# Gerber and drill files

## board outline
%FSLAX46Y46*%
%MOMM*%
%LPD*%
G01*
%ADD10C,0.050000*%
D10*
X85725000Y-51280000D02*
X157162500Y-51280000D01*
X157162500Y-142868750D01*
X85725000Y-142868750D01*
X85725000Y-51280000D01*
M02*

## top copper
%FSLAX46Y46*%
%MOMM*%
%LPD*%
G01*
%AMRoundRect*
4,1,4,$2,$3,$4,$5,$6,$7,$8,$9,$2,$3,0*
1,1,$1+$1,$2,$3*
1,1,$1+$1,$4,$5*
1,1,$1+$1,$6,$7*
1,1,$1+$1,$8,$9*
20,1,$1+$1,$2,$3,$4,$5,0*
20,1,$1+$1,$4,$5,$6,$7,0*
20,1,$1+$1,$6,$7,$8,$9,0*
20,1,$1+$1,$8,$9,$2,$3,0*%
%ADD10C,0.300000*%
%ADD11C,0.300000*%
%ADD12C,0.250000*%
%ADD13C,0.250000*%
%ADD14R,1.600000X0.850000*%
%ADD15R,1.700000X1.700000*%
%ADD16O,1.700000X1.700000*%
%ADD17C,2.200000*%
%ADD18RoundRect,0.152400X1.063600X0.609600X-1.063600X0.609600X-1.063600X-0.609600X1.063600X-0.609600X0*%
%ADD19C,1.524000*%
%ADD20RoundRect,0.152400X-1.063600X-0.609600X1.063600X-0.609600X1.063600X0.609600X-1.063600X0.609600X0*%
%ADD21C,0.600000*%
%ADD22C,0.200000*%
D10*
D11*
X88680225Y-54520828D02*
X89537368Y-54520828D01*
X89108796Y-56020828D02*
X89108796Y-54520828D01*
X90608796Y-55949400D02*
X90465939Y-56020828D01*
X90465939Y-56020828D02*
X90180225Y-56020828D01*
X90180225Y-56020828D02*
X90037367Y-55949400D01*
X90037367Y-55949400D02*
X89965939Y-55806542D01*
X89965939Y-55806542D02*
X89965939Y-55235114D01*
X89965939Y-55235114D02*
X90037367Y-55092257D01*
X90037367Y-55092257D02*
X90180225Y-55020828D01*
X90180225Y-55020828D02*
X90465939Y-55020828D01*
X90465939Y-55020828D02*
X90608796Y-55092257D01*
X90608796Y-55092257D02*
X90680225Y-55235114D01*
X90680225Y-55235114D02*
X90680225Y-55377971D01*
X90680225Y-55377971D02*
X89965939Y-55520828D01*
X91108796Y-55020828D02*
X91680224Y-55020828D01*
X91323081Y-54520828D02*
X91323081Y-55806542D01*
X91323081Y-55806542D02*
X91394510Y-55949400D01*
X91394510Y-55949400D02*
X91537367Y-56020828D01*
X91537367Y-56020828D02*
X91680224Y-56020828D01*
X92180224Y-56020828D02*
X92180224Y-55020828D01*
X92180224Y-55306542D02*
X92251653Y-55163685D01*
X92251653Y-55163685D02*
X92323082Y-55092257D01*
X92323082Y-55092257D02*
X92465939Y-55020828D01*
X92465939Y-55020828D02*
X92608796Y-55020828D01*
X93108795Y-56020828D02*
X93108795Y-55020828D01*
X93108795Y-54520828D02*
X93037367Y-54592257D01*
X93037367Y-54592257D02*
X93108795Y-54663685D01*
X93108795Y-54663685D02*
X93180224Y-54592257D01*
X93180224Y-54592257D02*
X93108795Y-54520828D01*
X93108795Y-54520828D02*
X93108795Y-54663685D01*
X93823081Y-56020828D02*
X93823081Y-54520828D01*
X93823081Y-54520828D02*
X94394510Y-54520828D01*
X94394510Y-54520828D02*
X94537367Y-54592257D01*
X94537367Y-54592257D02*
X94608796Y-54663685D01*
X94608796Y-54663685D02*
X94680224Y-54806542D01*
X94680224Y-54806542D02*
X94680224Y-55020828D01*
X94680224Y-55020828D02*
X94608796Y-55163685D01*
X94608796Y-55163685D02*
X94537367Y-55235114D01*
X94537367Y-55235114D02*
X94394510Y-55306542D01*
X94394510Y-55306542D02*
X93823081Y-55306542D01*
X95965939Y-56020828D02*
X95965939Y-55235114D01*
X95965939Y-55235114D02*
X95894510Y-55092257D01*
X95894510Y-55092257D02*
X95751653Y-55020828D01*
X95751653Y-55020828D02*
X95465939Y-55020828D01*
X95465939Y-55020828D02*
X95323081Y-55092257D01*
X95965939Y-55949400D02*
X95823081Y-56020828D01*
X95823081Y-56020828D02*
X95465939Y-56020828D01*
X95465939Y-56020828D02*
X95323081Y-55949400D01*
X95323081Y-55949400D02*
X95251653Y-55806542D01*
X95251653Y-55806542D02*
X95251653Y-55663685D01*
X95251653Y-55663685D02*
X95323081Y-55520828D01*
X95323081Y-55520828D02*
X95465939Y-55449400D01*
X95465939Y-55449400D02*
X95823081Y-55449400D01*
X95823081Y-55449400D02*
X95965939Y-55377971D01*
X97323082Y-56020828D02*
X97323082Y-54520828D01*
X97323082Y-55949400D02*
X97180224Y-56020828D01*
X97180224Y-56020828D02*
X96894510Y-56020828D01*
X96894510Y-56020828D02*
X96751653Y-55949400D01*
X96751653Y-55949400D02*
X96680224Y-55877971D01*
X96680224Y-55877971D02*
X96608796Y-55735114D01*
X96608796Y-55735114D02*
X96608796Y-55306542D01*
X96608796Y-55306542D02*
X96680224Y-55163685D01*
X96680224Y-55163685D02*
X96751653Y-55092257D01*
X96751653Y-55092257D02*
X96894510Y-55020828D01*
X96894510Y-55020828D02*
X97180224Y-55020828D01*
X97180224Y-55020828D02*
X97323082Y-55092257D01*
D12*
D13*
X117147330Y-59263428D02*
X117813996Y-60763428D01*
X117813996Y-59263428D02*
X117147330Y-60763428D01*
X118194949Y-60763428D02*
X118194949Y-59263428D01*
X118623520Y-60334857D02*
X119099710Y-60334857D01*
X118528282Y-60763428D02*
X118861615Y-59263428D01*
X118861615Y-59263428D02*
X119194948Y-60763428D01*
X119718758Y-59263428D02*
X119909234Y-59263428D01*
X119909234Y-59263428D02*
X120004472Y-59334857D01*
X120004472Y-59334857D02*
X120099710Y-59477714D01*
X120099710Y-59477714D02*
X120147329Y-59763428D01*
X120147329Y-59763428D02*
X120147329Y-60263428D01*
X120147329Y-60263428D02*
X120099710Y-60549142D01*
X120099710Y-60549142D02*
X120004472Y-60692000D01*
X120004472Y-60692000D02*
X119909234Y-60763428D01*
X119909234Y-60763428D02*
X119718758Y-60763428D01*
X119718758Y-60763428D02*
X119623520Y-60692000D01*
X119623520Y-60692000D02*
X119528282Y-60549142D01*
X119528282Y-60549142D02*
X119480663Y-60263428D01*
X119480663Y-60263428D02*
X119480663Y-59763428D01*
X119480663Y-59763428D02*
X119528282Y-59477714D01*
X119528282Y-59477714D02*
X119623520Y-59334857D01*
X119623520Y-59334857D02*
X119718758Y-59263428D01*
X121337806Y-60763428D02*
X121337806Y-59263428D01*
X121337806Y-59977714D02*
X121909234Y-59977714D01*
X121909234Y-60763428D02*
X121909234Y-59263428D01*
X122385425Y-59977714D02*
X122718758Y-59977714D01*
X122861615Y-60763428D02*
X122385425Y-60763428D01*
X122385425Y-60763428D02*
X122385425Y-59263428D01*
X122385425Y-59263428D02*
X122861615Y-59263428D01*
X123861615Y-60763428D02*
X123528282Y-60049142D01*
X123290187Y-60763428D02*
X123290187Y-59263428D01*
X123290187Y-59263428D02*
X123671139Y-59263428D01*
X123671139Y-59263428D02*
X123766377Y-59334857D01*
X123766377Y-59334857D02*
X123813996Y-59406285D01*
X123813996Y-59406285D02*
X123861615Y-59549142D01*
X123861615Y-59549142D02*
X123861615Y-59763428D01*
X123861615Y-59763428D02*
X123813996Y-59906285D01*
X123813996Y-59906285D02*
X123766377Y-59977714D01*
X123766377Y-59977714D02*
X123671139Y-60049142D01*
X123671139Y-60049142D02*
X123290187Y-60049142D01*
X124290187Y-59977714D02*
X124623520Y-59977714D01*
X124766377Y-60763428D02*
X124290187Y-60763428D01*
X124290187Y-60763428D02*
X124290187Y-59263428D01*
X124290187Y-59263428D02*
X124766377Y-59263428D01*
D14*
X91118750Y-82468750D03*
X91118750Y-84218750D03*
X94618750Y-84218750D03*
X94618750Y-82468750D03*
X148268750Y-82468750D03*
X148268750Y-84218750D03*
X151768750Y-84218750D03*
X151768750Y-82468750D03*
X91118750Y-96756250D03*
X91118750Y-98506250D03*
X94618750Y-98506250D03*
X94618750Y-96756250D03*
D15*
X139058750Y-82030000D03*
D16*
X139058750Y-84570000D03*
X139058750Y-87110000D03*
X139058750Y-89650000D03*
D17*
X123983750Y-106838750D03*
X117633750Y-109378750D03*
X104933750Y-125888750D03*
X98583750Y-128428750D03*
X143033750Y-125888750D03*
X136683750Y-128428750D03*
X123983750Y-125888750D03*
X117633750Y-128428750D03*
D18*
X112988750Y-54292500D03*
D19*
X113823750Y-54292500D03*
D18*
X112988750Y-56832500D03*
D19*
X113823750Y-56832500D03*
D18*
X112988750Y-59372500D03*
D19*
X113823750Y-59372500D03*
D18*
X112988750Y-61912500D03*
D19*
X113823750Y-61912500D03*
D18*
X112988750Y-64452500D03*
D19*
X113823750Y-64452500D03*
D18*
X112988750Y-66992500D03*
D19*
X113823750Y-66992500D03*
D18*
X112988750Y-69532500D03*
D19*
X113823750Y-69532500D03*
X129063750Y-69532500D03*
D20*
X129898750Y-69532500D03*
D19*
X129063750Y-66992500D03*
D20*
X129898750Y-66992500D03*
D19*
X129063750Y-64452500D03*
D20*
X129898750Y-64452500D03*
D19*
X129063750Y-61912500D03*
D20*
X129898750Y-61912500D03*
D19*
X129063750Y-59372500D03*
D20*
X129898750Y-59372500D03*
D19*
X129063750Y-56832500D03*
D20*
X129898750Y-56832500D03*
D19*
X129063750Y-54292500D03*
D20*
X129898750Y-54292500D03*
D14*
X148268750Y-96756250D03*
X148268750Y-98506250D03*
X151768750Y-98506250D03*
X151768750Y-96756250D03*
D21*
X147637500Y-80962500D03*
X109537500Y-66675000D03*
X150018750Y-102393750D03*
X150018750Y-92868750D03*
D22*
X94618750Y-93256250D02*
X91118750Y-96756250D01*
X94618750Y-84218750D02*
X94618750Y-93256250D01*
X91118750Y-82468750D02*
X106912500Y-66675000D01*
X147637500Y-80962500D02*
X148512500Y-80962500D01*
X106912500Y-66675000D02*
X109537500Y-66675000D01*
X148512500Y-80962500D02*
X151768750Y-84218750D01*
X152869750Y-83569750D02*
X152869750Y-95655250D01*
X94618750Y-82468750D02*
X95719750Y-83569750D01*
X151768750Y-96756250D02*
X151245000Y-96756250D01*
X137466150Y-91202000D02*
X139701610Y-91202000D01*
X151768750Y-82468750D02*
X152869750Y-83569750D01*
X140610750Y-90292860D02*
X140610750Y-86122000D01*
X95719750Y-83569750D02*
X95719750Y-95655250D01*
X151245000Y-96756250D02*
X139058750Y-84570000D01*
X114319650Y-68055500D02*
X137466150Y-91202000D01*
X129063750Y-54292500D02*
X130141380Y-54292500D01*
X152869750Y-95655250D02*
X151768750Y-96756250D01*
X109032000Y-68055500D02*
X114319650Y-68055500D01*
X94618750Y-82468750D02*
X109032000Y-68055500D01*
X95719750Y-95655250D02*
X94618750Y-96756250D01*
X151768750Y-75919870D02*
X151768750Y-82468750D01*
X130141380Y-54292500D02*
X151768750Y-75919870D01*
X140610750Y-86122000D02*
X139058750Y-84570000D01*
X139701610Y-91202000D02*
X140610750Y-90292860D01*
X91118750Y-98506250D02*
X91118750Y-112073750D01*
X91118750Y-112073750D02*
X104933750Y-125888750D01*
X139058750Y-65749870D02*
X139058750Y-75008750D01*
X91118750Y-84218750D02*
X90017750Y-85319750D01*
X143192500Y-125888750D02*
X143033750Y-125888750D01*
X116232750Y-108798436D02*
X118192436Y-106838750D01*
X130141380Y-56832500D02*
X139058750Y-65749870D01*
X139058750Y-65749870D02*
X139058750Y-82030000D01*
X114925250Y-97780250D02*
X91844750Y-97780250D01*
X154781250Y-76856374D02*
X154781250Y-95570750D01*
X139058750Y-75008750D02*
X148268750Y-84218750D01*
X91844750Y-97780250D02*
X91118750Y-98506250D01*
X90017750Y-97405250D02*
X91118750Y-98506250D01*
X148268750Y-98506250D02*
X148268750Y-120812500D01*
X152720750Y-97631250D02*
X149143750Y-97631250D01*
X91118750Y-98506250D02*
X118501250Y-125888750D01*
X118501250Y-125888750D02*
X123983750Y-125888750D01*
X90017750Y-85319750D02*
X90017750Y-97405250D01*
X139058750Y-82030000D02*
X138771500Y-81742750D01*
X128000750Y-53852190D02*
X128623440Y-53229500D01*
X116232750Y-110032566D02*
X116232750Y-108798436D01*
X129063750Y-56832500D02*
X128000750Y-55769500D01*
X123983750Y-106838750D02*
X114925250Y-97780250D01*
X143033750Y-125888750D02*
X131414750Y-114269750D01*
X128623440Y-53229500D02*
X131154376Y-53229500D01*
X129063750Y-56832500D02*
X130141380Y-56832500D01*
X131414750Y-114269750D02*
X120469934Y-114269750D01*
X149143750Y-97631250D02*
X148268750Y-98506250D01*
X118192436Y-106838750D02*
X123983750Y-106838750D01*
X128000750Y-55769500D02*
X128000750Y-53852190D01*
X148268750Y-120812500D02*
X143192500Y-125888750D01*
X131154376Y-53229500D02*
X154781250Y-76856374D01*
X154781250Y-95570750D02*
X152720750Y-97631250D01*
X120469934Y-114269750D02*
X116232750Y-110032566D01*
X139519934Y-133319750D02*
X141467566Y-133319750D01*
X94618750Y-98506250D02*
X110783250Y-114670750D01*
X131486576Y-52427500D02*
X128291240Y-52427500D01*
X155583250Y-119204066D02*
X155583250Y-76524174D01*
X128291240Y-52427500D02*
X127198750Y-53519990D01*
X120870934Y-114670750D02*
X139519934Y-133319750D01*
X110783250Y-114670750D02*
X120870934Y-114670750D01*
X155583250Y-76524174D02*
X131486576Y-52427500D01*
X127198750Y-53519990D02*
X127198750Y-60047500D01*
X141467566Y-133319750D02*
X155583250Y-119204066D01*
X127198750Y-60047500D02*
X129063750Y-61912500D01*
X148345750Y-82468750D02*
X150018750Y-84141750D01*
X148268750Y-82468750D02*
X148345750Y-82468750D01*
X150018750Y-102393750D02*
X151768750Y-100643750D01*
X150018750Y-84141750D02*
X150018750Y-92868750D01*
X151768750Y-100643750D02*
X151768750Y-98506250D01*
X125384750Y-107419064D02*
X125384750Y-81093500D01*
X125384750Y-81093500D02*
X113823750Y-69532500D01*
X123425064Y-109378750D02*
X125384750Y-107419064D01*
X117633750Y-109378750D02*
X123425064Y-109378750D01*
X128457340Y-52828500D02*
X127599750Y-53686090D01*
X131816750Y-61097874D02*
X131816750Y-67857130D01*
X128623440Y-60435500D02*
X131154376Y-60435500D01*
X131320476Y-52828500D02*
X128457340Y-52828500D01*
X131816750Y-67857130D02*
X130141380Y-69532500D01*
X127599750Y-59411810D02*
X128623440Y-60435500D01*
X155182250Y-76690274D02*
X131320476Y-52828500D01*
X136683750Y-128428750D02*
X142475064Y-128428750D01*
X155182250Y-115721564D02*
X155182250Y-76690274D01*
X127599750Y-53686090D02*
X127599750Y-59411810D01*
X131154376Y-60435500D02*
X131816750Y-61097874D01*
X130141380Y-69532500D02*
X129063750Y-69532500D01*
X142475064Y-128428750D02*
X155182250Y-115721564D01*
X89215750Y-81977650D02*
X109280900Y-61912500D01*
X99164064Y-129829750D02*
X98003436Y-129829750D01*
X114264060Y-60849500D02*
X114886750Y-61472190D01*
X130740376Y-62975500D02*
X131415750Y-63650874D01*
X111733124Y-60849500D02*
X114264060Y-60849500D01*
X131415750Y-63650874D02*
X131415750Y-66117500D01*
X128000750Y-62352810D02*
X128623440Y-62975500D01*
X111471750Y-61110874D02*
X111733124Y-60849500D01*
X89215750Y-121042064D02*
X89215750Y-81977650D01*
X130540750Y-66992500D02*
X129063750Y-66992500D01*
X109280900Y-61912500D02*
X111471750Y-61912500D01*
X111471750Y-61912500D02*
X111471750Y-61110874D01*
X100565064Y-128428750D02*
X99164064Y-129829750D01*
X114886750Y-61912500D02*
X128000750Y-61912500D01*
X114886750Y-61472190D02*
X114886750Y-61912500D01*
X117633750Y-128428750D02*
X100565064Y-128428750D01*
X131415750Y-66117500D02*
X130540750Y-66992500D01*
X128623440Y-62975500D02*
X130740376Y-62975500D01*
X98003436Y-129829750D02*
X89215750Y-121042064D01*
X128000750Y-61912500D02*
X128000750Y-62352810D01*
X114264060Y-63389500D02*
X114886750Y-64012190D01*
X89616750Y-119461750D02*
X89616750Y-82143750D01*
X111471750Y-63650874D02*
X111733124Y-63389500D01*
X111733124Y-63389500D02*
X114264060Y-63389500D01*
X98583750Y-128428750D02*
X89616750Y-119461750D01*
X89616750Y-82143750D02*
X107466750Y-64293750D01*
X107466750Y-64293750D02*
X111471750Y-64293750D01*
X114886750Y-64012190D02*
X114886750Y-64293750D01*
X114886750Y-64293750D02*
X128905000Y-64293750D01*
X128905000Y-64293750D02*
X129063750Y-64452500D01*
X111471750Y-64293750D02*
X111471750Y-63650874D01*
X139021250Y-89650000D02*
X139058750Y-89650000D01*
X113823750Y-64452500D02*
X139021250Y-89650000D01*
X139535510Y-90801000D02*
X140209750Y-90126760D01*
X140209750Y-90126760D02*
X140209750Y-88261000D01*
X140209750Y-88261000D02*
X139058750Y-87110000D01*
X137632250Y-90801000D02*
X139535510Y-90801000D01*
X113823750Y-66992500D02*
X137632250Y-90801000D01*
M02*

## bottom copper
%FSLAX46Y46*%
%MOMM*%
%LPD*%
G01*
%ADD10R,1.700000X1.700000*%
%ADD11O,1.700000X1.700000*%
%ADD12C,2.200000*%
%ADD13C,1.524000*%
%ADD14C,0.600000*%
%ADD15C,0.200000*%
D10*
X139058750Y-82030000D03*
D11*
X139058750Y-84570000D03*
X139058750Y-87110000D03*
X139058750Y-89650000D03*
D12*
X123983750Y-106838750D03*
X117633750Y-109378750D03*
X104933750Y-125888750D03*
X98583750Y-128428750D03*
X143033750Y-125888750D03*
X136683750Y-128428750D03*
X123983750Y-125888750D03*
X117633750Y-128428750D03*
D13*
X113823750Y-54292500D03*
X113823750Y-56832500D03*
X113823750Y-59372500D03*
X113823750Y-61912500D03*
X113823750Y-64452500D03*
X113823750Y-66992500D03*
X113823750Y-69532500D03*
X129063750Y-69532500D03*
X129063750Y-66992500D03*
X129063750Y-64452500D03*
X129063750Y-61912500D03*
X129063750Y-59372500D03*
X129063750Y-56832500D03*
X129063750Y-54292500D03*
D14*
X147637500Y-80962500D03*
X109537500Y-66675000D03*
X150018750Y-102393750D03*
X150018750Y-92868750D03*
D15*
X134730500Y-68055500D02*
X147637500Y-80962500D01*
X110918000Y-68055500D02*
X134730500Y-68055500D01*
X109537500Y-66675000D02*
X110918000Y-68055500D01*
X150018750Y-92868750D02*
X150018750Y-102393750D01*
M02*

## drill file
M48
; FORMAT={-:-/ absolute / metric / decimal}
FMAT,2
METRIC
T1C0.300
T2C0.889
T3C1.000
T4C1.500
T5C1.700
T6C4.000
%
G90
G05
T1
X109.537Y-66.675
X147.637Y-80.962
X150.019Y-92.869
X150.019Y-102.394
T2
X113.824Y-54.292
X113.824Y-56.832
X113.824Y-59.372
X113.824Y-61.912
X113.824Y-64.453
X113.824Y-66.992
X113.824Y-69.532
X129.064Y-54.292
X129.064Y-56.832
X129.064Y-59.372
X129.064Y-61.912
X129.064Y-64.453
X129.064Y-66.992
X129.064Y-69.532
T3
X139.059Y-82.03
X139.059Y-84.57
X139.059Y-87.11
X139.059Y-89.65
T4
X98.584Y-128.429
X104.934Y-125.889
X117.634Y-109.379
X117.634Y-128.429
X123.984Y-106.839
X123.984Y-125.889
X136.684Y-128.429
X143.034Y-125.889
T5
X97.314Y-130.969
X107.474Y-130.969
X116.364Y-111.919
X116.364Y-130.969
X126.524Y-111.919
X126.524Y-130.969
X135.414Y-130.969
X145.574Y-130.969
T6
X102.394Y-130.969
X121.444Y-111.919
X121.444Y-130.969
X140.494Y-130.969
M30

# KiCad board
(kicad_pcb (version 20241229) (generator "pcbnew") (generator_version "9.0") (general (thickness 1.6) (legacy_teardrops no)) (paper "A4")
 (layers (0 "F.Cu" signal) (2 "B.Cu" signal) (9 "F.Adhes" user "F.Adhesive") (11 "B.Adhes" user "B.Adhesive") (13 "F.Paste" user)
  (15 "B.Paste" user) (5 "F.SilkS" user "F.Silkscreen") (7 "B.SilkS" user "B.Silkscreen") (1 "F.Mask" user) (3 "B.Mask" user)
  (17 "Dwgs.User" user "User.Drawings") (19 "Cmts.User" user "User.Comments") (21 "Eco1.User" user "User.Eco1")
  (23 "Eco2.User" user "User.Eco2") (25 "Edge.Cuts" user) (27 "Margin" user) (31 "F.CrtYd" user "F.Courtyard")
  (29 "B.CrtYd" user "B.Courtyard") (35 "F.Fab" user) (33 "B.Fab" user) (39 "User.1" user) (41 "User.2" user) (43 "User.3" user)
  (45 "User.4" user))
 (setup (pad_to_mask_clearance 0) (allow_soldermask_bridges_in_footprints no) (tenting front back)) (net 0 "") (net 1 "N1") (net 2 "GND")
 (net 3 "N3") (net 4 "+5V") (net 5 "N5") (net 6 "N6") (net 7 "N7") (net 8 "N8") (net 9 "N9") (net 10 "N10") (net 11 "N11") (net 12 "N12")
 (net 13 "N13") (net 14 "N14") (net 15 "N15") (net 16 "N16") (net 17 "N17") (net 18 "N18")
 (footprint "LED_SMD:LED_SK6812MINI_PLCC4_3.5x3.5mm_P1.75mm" (layer "F.Cu") (at 92.86875 83.34375)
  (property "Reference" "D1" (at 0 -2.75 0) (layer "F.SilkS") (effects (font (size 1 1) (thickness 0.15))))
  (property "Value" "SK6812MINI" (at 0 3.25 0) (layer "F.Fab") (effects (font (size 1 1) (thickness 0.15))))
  (pad "1" smd rect (at -1.75 -0.875) (size 1.6 0.85) (layers "F.Cu" "F.Mask" "F.Paste") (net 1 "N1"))
  (pad "2" smd rect (at -1.75 0.875) (size 1.6 0.85) (layers "F.Cu" "F.Mask" "F.Paste") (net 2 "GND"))
  (pad "3" smd rect (at 1.75 0.875) (size 1.6 0.85) (layers "F.Cu" "F.Mask" "F.Paste") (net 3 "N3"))
  (pad "4" smd rect (at 1.75 -0.875) (size 1.6 0.85) (layers "F.Cu" "F.Mask" "F.Paste") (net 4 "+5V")))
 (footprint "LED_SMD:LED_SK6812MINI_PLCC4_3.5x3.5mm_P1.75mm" (layer "F.Cu") (at 150.01875 83.34375)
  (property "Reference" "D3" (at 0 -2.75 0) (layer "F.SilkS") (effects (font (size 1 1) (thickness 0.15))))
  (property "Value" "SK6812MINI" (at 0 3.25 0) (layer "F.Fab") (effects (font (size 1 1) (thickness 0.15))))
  (pad "1" smd rect (at -1.75 -0.875) (size 1.6 0.85) (layers "F.Cu" "F.Mask" "F.Paste") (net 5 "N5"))
  (pad "2" smd rect (at -1.75 0.875) (size 1.6 0.85) (layers "F.Cu" "F.Mask" "F.Paste") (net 2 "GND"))
  (pad "3" smd rect (at 1.75 0.875) (size 1.6 0.85) (layers "F.Cu" "F.Mask" "F.Paste") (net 1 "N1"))
  (pad "4" smd rect (at 1.75 -0.875) (size 1.6 0.85) (layers "F.Cu" "F.Mask" "F.Paste") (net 4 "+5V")))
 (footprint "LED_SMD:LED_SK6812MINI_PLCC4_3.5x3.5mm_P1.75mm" (layer "F.Cu") (at 92.86875 97.63125)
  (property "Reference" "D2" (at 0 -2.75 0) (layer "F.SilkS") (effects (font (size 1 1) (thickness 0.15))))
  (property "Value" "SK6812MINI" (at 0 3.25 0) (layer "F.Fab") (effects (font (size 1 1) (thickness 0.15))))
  (pad "1" smd rect (at -1.75 -0.875) (size 1.6 0.85) (layers "F.Cu" "F.Mask" "F.Paste") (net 3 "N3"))
  (pad "2" smd rect (at -1.75 0.875) (size 1.6 0.85) (layers "F.Cu" "F.Mask" "F.Paste") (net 2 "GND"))
  (pad "3" smd rect (at 1.75 0.875) (size 1.6 0.85) (layers "F.Cu" "F.Mask" "F.Paste") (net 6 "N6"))
  (pad "4" smd rect (at 1.75 -0.875) (size 1.6 0.85) (layers "F.Cu" "F.Mask" "F.Paste") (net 4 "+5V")))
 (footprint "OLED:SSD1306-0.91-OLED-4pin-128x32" (layer "F.Cu") (at 102.55875 79.84)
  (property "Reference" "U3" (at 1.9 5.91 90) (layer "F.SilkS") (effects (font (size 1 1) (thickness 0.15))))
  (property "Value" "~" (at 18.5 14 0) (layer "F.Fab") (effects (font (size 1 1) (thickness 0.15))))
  (pad "1" thru_hole rect (at 36.5 2.19) (size 1.7 1.7) (drill 1) (layers "*.Cu" "*.Mask") (remove_unused_layers no) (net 2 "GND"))
  (pad "2" thru_hole oval (at 36.5 4.73) (size 1.7 1.7) (drill 1) (layers "*.Cu" "*.Mask") (remove_unused_layers no) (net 4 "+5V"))
  (pad "3" thru_hole oval (at 36.5 7.27) (size 1.7 1.7) (drill 1) (layers "*.Cu" "*.Mask") (remove_unused_layers no) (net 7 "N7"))
  (pad "4" thru_hole oval (at 36.5 9.81) (size 1.7 1.7) (drill 1) (layers "*.Cu" "*.Mask") (remove_unused_layers no) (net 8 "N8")))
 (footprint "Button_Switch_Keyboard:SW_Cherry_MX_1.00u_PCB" (layer "F.Cu") (at 123.98375 106.83875)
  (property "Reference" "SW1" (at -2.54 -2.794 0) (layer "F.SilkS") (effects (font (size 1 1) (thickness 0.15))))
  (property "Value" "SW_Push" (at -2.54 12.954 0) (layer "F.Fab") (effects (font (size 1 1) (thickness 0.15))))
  (pad "" np_thru_hole circle (at -7.62 5.08) (size 1.7 1.7) (drill 1.7) (layers "*.Cu" "*.Mask"))
  (pad "" np_thru_hole circle (at -2.54 5.08) (size 4 4) (drill 4) (layers "*.Cu" "*.Mask"))
  (pad "" np_thru_hole circle (at 2.54 5.08) (size 1.7 1.7) (drill 1.7) (layers "*.Cu" "*.Mask"))
  (pad "1" thru_hole circle (at 0 0) (size 2.2 2.2) (drill 1.5) (layers "*.Cu" "*.Mask") (remove_unused_layers no) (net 2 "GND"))
  (pad "2" thru_hole circle (at -6.35 2.54) (size 2.2 2.2) (drill 1.5) (layers "*.Cu" "*.Mask") (remove_unused_layers no) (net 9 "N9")))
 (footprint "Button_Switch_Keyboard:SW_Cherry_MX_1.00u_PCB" (layer "F.Cu") (at 104.93375 125.88875)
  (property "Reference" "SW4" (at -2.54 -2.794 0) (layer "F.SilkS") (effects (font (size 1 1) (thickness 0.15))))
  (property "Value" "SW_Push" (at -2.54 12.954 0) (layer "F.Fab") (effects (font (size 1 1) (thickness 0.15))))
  (pad "" np_thru_hole circle (at -7.62 5.08) (size 1.7 1.7) (drill 1.7) (layers "*.Cu" "*.Mask"))
  (pad "" np_thru_hole circle (at -2.54 5.08) (size 4 4) (drill 4) (layers "*.Cu" "*.Mask"))
  (pad "" np_thru_hole circle (at 2.54 5.08) (size 1.7 1.7) (drill 1.7) (layers "*.Cu" "*.Mask"))
  (pad "1" thru_hole circle (at 0 0) (size 2.2 2.2) (drill 1.5) (layers "*.Cu" "*.Mask") (remove_unused_layers no) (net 2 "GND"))
  (pad "2" thru_hole circle (at -6.35 2.54) (size 2.2 2.2) (drill 1.5) (layers "*.Cu" "*.Mask") (remove_unused_layers no) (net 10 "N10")))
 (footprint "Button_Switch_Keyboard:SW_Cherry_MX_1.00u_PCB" (layer "F.Cu") (at 143.03375 125.88875)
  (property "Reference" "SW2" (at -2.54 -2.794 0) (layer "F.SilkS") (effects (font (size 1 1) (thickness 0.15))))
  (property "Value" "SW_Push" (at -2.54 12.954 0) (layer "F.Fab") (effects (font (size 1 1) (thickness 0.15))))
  (pad "" np_thru_hole circle (at -7.62 5.08) (size 1.7 1.7) (drill 1.7) (layers "*.Cu" "*.Mask"))
  (pad "" np_thru_hole circle (at -2.54 5.08) (size 4 4) (drill 4) (layers "*.Cu" "*.Mask"))
  (pad "" np_thru_hole circle (at 2.54 5.08) (size 1.7 1.7) (drill 1.7) (layers "*.Cu" "*.Mask"))
  (pad "1" thru_hole circle (at 0 0) (size 2.2 2.2) (drill 1.5) (layers "*.Cu" "*.Mask") (remove_unused_layers no) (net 2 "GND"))
  (pad "2" thru_hole circle (at -6.35 2.54) (size 2.2 2.2) (drill 1.5) (layers "*.Cu" "*.Mask") (remove_unused_layers no) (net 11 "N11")))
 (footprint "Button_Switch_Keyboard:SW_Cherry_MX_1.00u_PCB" (layer "F.Cu") (at 123.98375 125.88875)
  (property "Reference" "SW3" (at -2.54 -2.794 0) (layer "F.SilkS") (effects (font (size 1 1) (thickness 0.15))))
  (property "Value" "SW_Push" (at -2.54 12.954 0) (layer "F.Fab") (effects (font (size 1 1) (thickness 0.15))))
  (pad "" np_thru_hole circle (at -7.62 5.08) (size 1.7 1.7) (drill 1.7) (layers "*.Cu" "*.Mask"))
  (pad "" np_thru_hole circle (at -2.54 5.08) (size 4 4) (drill 4) (layers "*.Cu" "*.Mask"))
  (pad "" np_thru_hole circle (at 2.54 5.08) (size 1.7 1.7) (drill 1.7) (layers "*.Cu" "*.Mask"))
  (pad "1" thru_hole circle (at 0 0) (size 2.2 2.2) (drill 1.5) (layers "*.Cu" "*.Mask") (remove_unused_layers no) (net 2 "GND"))
  (pad "2" thru_hole circle (at -6.35 2.54) (size 2.2 2.2) (drill 1.5) (layers "*.Cu" "*.Mask") (remove_unused_layers no) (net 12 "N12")))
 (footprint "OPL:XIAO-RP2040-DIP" (layer "F.Cu") (at 121.44375 61.9125)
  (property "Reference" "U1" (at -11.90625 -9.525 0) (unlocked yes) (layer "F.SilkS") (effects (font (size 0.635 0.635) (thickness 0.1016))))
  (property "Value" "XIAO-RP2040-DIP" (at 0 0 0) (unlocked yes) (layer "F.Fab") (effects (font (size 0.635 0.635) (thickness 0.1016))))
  (pad "1" smd roundrect (at -8.455 -7.62 180) (size 2.432 1.524) (layers "F.Cu" "F.Mask") (roundrect_rratio 0.1) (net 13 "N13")
   (thermal_bridge_angle 45))
  (pad "1" thru_hole circle (at -7.62 -7.62 180) (size 1.524 1.524) (drill 0.889) (layers "*.Cu" "*.Mask") (remove_unused_layers no)
   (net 13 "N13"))
  (pad "2" smd roundrect (at -8.455 -5.08 180) (size 2.432 1.524) (layers "F.Cu" "F.Mask") (roundrect_rratio 0.1) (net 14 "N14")
   (thermal_bridge_angle 45))
  (pad "2" thru_hole circle (at -7.62 -5.08 180) (size 1.524 1.524) (drill 0.889) (layers "*.Cu" "*.Mask") (remove_unused_layers no)
   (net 14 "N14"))
  (pad "3" smd roundrect (at -8.455 -2.54 180) (size 2.432 1.524) (layers "F.Cu" "F.Mask") (roundrect_rratio 0.1) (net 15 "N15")
   (thermal_bridge_angle 45))
  (pad "3" thru_hole circle (at -7.62 -2.54 180) (size 1.524 1.524) (drill 0.889) (layers "*.Cu" "*.Mask") (remove_unused_layers no)
   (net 15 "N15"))
  (pad "4" smd roundrect (at -8.455 0 180) (size 2.432 1.524) (layers "F.Cu" "F.Mask") (roundrect_rratio 0.1) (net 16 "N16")
   (thermal_bridge_angle 45))
  (pad "4" thru_hole circle (at -7.62 0 180) (size 1.524 1.524) (drill 0.889) (layers "*.Cu" "*.Mask") (remove_unused_layers no)
   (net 16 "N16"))
  (pad "5" smd roundrect (at -8.455 2.54 180) (size 2.432 1.524) (layers "F.Cu" "F.Mask") (roundrect_rratio 0.1) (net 8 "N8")
   (thermal_bridge_angle 45))
  (pad "5" thru_hole circle (at -7.62 2.54 180) (size 1.524 1.524) (drill 0.889) (layers "*.Cu" "*.Mask") (remove_unused_layers no)
   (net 8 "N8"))
  (pad "6" smd roundrect (at -8.455 5.08 180) (size 2.432 1.524) (layers "F.Cu" "F.Mask") (roundrect_rratio 0.1) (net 7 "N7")
   (thermal_bridge_angle 45))
  (pad "6" thru_hole circle (at -7.62 5.08 180) (size 1.524 1.524) (drill 0.889) (layers "*.Cu" "*.Mask") (remove_unused_layers no)
   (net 7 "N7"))
  (pad "7" smd roundrect (at -8.455 7.62 180) (size 2.432 1.524) (layers "F.Cu" "F.Mask") (roundrect_rratio 0.1) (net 9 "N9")
   (thermal_bridge_angle 45))
  (pad "7" thru_hole circle (at -7.62 7.62 180) (size 1.524 1.524) (drill 0.889) (layers "*.Cu" "*.Mask") (remove_unused_layers no)
   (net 9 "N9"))
  (pad "8" thru_hole circle (at 7.62 7.62) (size 1.524 1.524) (drill 0.889) (layers "*.Cu" "*.Mask") (remove_unused_layers no)
   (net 11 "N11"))
  (pad "8" smd roundrect (at 8.455 7.62) (size 2.432 1.524) (layers "F.Cu" "F.Mask") (roundrect_rratio 0.1) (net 11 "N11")
   (thermal_bridge_angle 45))
  (pad "9" thru_hole circle (at 7.62 5.08) (size 1.524 1.524) (drill 0.889) (layers "*.Cu" "*.Mask") (remove_unused_layers no)
   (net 12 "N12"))
  (pad "9" smd roundrect (at 8.455 5.08) (size 2.432 1.524) (layers "F.Cu" "F.Mask") (roundrect_rratio 0.1) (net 12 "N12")
   (thermal_bridge_angle 45))
  (pad "10" thru_hole circle (at 7.62 2.54) (size 1.524 1.524) (drill 0.889) (layers "*.Cu" "*.Mask") (remove_unused_layers no)
   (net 10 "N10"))
  (pad "10" smd roundrect (at 8.455 2.54) (size 2.432 1.524) (layers "F.Cu" "F.Mask") (roundrect_rratio 0.1) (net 10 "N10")
   (thermal_bridge_angle 45))
  (pad "11" thru_hole circle (at 7.62 0) (size 1.524 1.524) (drill 0.889) (layers "*.Cu" "*.Mask") (remove_unused_layers no) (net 6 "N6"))
  (pad "11" smd roundrect (at 8.455 0) (size 2.432 1.524) (layers "F.Cu" "F.Mask") (roundrect_rratio 0.1) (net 6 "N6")
   (thermal_bridge_angle 45))
  (pad "12" thru_hole circle (at 7.62 -2.54) (size 1.524 1.524) (drill 0.889) (layers "*.Cu" "*.Mask") (remove_unused_layers no)
   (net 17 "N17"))
  (pad "12" smd roundrect (at 8.455 -2.54) (size 2.432 1.524) (layers "F.Cu" "F.Mask") (roundrect_rratio 0.1) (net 17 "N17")
   (thermal_bridge_angle 45))
  (pad "13" thru_hole circle (at 7.62 -5.08) (size 1.524 1.524) (drill 0.889) (layers "*.Cu" "*.Mask") (remove_unused_layers no)
   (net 2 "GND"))
  (pad "13" smd roundrect (at 8.455 -5.08) (size 2.432 1.524) (layers "F.Cu" "F.Mask") (roundrect_rratio 0.1) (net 2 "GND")
   (thermal_bridge_angle 45))
  (pad "14" thru_hole circle (at 7.62 -7.62) (size 1.524 1.524) (drill 0.889) (layers "*.Cu" "*.Mask") (remove_unused_layers no)
   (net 4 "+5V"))
  (pad "14" smd roundrect (at 8.455 -7.62) (size 2.432 1.524) (layers "F.Cu" "F.Mask") (roundrect_rratio 0.1) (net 4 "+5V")
   (thermal_bridge_angle 45)))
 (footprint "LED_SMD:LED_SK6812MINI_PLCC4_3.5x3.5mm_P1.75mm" (layer "F.Cu") (at 150.01875 97.63125)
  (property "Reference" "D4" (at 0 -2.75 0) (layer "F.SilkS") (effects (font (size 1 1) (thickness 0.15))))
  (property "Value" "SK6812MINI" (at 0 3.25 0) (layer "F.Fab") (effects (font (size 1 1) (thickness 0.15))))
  (pad "1" smd rect (at -1.75 -0.875) (size 1.6 0.85) (layers "F.Cu" "F.Mask" "F.Paste") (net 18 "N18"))
  (pad "2" smd rect (at -1.75 0.875) (size 1.6 0.85) (layers "F.Cu" "F.Mask" "F.Paste") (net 2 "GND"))
  (pad "3" smd rect (at 1.75 0.875) (size 1.6 0.85) (layers "F.Cu" "F.Mask" "F.Paste") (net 5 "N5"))
  (pad "4" smd rect (at 1.75 -0.875) (size 1.6 0.85) (layers "F.Cu" "F.Mask" "F.Paste") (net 4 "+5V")))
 (gr_rect (start 85.725 51.28) (end 157.1625 142.86875) (stroke (width 0.05) (type default)) (fill no) (layer "Edge.Cuts"))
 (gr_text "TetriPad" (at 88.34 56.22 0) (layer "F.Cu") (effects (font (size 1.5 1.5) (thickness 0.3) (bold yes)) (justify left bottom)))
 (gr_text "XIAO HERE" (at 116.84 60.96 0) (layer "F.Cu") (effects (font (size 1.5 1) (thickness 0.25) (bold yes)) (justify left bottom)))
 (segment (start 94.61875 93.25625) (end 91.11875 96.75625) (width 0.2) (layer "F.Cu") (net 3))
 (segment (start 94.61875 84.21875) (end 94.61875 93.25625) (width 0.2) (layer "F.Cu") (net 3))
 (segment (start 91.11875 82.46875) (end 106.9125 66.675) (width 0.2) (layer "F.Cu") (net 1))
 (segment (start 147.6375 80.9625) (end 148.5125 80.9625) (width 0.2) (layer "F.Cu") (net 1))
 (segment (start 106.9125 66.675) (end 109.5375 66.675) (width 0.2) (layer "F.Cu") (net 1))
 (segment (start 148.5125 80.9625) (end 151.76875 84.21875) (width 0.2) (layer "F.Cu") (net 1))
 (via (at 147.6375 80.9625) (size 0.6) (drill 0.3) (layers "F.Cu" "B.Cu") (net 1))
 (via (at 109.5375 66.675) (size 0.6) (drill 0.3) (layers "F.Cu" "B.Cu") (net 1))
 (segment (start 134.7305 68.0555) (end 147.6375 80.9625) (width 0.2) (layer "B.Cu") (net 1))
 (segment (start 110.918 68.0555) (end 134.7305 68.0555) (width 0.2) (layer "B.Cu") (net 1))
 (segment (start 109.5375 66.675) (end 110.918 68.0555) (width 0.2) (layer "B.Cu") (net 1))
 (segment (start 152.86975 83.56975) (end 152.86975 95.65525) (width 0.2) (layer "F.Cu") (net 4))
 (segment (start 94.61875 82.46875) (end 95.71975 83.56975) (width 0.2) (layer "F.Cu") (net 4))
 (segment (start 151.76875 96.75625) (end 151.245 96.75625) (width 0.2) (layer "F.Cu") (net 4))
 (segment (start 137.46615 91.202) (end 139.70161 91.202) (width 0.2) (layer "F.Cu") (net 4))
 (segment (start 151.76875 82.46875) (end 152.86975 83.56975) (width 0.2) (layer "F.Cu") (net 4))
 (segment (start 140.61075 90.29286) (end 140.61075 86.122) (width 0.2) (layer "F.Cu") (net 4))
 (segment (start 95.71975 83.56975) (end 95.71975 95.65525) (width 0.2) (layer "F.Cu") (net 4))
 (segment (start 151.245 96.75625) (end 139.05875 84.57) (width 0.2) (layer "F.Cu") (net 4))
 (segment (start 114.31965 68.0555) (end 137.46615 91.202) (width 0.2) (layer "F.Cu") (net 4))
 (segment (start 129.06375 54.2925) (end 130.14138 54.2925) (width 0.2) (layer "F.Cu") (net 4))
 (segment (start 152.86975 95.65525) (end 151.76875 96.75625) (width 0.2) (layer "F.Cu") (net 4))
 (segment (start 109.032 68.0555) (end 114.31965 68.0555) (width 0.2) (layer "F.Cu") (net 4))
 (segment (start 94.61875 82.46875) (end 109.032 68.0555) (width 0.2) (layer "F.Cu") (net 4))
 (segment (start 95.71975 95.65525) (end 94.61875 96.75625) (width 0.2) (layer "F.Cu") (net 4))
 (segment (start 151.76875 75.91987) (end 151.76875 82.46875) (width 0.2) (layer "F.Cu") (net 4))
 (segment (start 130.14138 54.2925) (end 151.76875 75.91987) (width 0.2) (layer "F.Cu") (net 4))
 (segment (start 140.61075 86.122) (end 139.05875 84.57) (width 0.2) (layer "F.Cu") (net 4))
 (segment (start 139.70161 91.202) (end 140.61075 90.29286) (width 0.2) (layer "F.Cu") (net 4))
 (segment (start 91.11875 98.50625) (end 91.11875 112.07375) (width 0.2) (layer "F.Cu") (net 2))
 (segment (start 91.11875 112.07375) (end 104.93375 125.88875) (width 0.2) (layer "F.Cu") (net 2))
 (segment (start 139.05875 65.74987) (end 139.05875 75.00875) (width 0.2) (layer "F.Cu") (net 2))
 (segment (start 91.11875 84.21875) (end 90.01775 85.31975) (width 0.2) (layer "F.Cu") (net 2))
 (segment (start 143.1925 125.88875) (end 143.03375 125.88875) (width 0.2) (layer "F.Cu") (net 2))
 (segment (start 116.23275 108.798436) (end 118.192436 106.83875) (width 0.2) (layer "F.Cu") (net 2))
 (segment (start 130.14138 56.8325) (end 139.05875 65.74987) (width 0.2) (layer "F.Cu") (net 2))
 (segment (start 139.05875 65.74987) (end 139.05875 82.03) (width 0.2) (layer "F.Cu") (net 2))
 (segment (start 114.92525 97.78025) (end 91.84475 97.78025) (width 0.2) (layer "F.Cu") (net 2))
 (segment (start 154.78125 76.856374) (end 154.78125 95.57075) (width 0.2) (layer "F.Cu") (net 2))
 (segment (start 139.05875 75.00875) (end 148.26875 84.21875) (width 0.2) (layer "F.Cu") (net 2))
 (segment (start 91.84475 97.78025) (end 91.11875 98.50625) (width 0.2) (layer "F.Cu") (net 2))
 (segment (start 90.01775 97.40525) (end 91.11875 98.50625) (width 0.2) (layer "F.Cu") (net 2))
 (segment (start 148.26875 98.50625) (end 148.26875 120.8125) (width 0.2) (layer "F.Cu") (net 2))
 (segment (start 152.72075 97.63125) (end 149.14375 97.63125) (width 0.2) (layer "F.Cu") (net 2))
 (segment (start 91.11875 98.50625) (end 118.50125 125.88875) (width 0.2) (layer "F.Cu") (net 2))
 (segment (start 118.50125 125.88875) (end 123.98375 125.88875) (width 0.2) (layer "F.Cu") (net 2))
 (segment (start 90.01775 85.31975) (end 90.01775 97.40525) (width 0.2) (layer "F.Cu") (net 2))
 (segment (start 139.05875 82.03) (end 138.7715 81.74275) (width 0.2) (layer "F.Cu") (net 2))
 (segment (start 128.00075 53.85219) (end 128.62344 53.2295) (width 0.2) (layer "F.Cu") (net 2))
 (segment (start 116.23275 110.032566) (end 116.23275 108.798436) (width 0.2) (layer "F.Cu") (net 2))
 (segment (start 129.06375 56.8325) (end 128.00075 55.7695) (width 0.2) (layer "F.Cu") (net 2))
 (segment (start 123.98375 106.83875) (end 114.92525 97.78025) (width 0.2) (layer "F.Cu") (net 2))
 (segment (start 143.03375 125.88875) (end 131.41475 114.26975) (width 0.2) (layer "F.Cu") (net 2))
 (segment (start 128.62344 53.2295) (end 131.154376 53.2295) (width 0.2) (layer "F.Cu") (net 2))
 (segment (start 129.06375 56.8325) (end 130.14138 56.8325) (width 0.2) (layer "F.Cu") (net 2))
 (segment (start 131.41475 114.26975) (end 120.469934 114.26975) (width 0.2) (layer "F.Cu") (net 2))
 (segment (start 149.14375 97.63125) (end 148.26875 98.50625) (width 0.2) (layer "F.Cu") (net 2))
 (segment (start 118.192436 106.83875) (end 123.98375 106.83875) (width 0.2) (layer "F.Cu") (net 2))
 (segment (start 128.00075 55.7695) (end 128.00075 53.85219) (width 0.2) (layer "F.Cu") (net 2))
 (segment (start 148.26875 120.8125) (end 143.1925 125.88875) (width 0.2) (layer "F.Cu") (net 2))
 (segment (start 131.154376 53.2295) (end 154.78125 76.856374) (width 0.2) (layer "F.Cu") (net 2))
 (segment (start 154.78125 95.57075) (end 152.72075 97.63125) (width 0.2) (layer "F.Cu") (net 2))
 (segment (start 120.469934 114.26975) (end 116.23275 110.032566) (width 0.2) (layer "F.Cu") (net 2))
 (segment (start 139.519934 133.31975) (end 141.467566 133.31975) (width 0.2) (layer "F.Cu") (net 6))
 (segment (start 94.61875 98.50625) (end 110.78325 114.67075) (width 0.2) (layer "F.Cu") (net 6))
 (segment (start 131.486576 52.4275) (end 128.29124 52.4275) (width 0.2) (layer "F.Cu") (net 6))
 (segment (start 155.58325 119.204066) (end 155.58325 76.524174) (width 0.2) (layer "F.Cu") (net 6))
 (segment (start 128.29124 52.4275) (end 127.19875 53.51999) (width 0.2) (layer "F.Cu") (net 6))
 (segment (start 120.870934 114.67075) (end 139.519934 133.31975) (width 0.2) (layer "F.Cu") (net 6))
 (segment (start 110.78325 114.67075) (end 120.870934 114.67075) (width 0.2) (layer "F.Cu") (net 6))
 (segment (start 155.58325 76.524174) (end 131.486576 52.4275) (width 0.2) (layer "F.Cu") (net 6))
 (segment (start 127.19875 53.51999) (end 127.19875 60.0475) (width 0.2) (layer "F.Cu") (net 6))
 (segment (start 141.467566 133.31975) (end 155.58325 119.204066) (width 0.2) (layer "F.Cu") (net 6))
 (segment (start 127.19875 60.0475) (end 129.06375 61.9125) (width 0.2) (layer "F.Cu") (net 6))
 (segment (start 148.34575 82.46875) (end 150.01875 84.14175) (width 0.2) (layer "F.Cu") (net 5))
 (segment (start 148.26875 82.46875) (end 148.34575 82.46875) (width 0.2) (layer "F.Cu") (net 5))
 (segment (start 150.01875 102.39375) (end 151.76875 100.64375) (width 0.2) (layer "F.Cu") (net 5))
 (segment (start 150.01875 84.14175) (end 150.01875 92.86875) (width 0.2) (layer "F.Cu") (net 5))
 (segment (start 151.76875 100.64375) (end 151.76875 98.50625) (width 0.2) (layer "F.Cu") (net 5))
 (via (at 150.01875 102.39375) (size 0.6) (drill 0.3) (layers "F.Cu" "B.Cu") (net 5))
 (via (at 150.01875 92.86875) (size 0.6) (drill 0.3) (layers "F.Cu" "B.Cu") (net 5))
 (segment (start 150.01875 92.86875) (end 150.01875 102.39375) (width 0.2) (layer "B.Cu") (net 5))
 (segment (start 125.38475 107.419064) (end 125.38475 81.0935) (width 0.2) (layer "F.Cu") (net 9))
 (segment (start 125.38475 81.0935) (end 113.82375 69.5325) (width 0.2) (layer "F.Cu") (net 9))
 (segment (start 123.425064 109.37875) (end 125.38475 107.419064) (width 0.2) (layer "F.Cu") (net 9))
 (segment (start 117.63375 109.37875) (end 123.425064 109.37875) (width 0.2) (layer "F.Cu") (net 9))
 (segment (start 128.45734 52.8285) (end 127.59975 53.68609) (width 0.2) (layer "F.Cu") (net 11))
 (segment (start 131.81675 61.097874) (end 131.81675 67.85713) (width 0.2) (layer "F.Cu") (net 11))
 (segment (start 128.62344 60.4355) (end 131.154376 60.4355) (width 0.2) (layer "F.Cu") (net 11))
 (segment (start 131.320476 52.8285) (end 128.45734 52.8285) (width 0.2) (layer "F.Cu") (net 11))
 (segment (start 131.81675 67.85713) (end 130.14138 69.5325) (width 0.2) (layer "F.Cu") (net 11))
 (segment (start 127.59975 59.41181) (end 128.62344 60.4355) (width 0.2) (layer "F.Cu") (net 11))
 (segment (start 155.18225 76.690274) (end 131.320476 52.8285) (width 0.2) (layer "F.Cu") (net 11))
 (segment (start 136.68375 128.42875) (end 142.475064 128.42875) (width 0.2) (layer "F.Cu") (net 11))
 (segment (start 155.18225 115.721564) (end 155.18225 76.690274) (width 0.2) (layer "F.Cu") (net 11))
 (segment (start 127.59975 53.68609) (end 127.59975 59.41181) (width 0.2) (layer "F.Cu") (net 11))
 (segment (start 131.154376 60.4355) (end 131.81675 61.097874) (width 0.2) (layer "F.Cu") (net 11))
 (segment (start 130.14138 69.5325) (end 129.06375 69.5325) (width 0.2) (layer "F.Cu") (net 11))
 (segment (start 142.475064 128.42875) (end 155.18225 115.721564) (width 0.2) (layer "F.Cu") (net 11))
 (segment (start 89.21575 81.97765) (end 109.2809 61.9125) (width 0.2) (layer "F.Cu") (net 12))
 (segment (start 99.164064 129.82975) (end 98.003436 129.82975) (width 0.2) (layer "F.Cu") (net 12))
 (segment (start 114.26406 60.8495) (end 114.88675 61.47219) (width 0.2) (layer "F.Cu") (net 12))
 (segment (start 130.740376 62.9755) (end 131.41575 63.650874) (width 0.2) (layer "F.Cu") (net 12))
 (segment (start 111.733124 60.8495) (end 114.26406 60.8495) (width 0.2) (layer "F.Cu") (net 12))
 (segment (start 131.41575 63.650874) (end 131.41575 66.1175) (width 0.2) (layer "F.Cu") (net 12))
 (segment (start 128.00075 62.35281) (end 128.62344 62.9755) (width 0.2) (layer "F.Cu") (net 12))
 (segment (start 111.47175 61.110874) (end 111.733124 60.8495) (width 0.2) (layer "F.Cu") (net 12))
 (segment (start 89.21575 121.042064) (end 89.21575 81.97765) (width 0.2) (layer "F.Cu") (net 12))
 (segment (start 130.54075 66.9925) (end 129.06375 66.9925) (width 0.2) (layer "F.Cu") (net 12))
 (segment (start 109.2809 61.9125) (end 111.47175 61.9125) (width 0.2) (layer "F.Cu") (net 12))
 (segment (start 111.47175 61.9125) (end 111.47175 61.110874) (width 0.2) (layer "F.Cu") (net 12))
 (segment (start 100.565064 128.42875) (end 99.164064 129.82975) (width 0.2) (layer "F.Cu") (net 12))
 (segment (start 114.88675 61.9125) (end 128.00075 61.9125) (width 0.2) (layer "F.Cu") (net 12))
 (segment (start 114.88675 61.47219) (end 114.88675 61.9125) (width 0.2) (layer "F.Cu") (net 12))
 (segment (start 117.63375 128.42875) (end 100.565064 128.42875) (width 0.2) (layer "F.Cu") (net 12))
 (segment (start 131.41575 66.1175) (end 130.54075 66.9925) (width 0.2) (layer "F.Cu") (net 12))
 (segment (start 128.62344 62.9755) (end 130.740376 62.9755) (width 0.2) (layer "F.Cu") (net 12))
 (segment (start 98.003436 129.82975) (end 89.21575 121.042064) (width 0.2) (layer "F.Cu") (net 12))
 (segment (start 128.00075 61.9125) (end 128.00075 62.35281) (width 0.2) (layer "F.Cu") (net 12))
 (segment (start 114.26406 63.3895) (end 114.88675 64.01219) (width 0.2) (layer "F.Cu") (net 10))
 (segment (start 89.61675 119.46175) (end 89.61675 82.14375) (width 0.2) (layer "F.Cu") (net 10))
 (segment (start 111.47175 63.650874) (end 111.733124 63.3895) (width 0.2) (layer "F.Cu") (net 10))
 (segment (start 111.733124 63.3895) (end 114.26406 63.3895) (width 0.2) (layer "F.Cu") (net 10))
 (segment (start 98.58375 128.42875) (end 89.61675 119.46175) (width 0.2) (layer "F.Cu") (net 10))
 (segment (start 89.61675 82.14375) (end 107.46675 64.29375) (width 0.2) (layer "F.Cu") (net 10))
 (segment (start 107.46675 64.29375) (end 111.47175 64.29375) (width 0.2) (layer "F.Cu") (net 10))
 (segment (start 114.88675 64.01219) (end 114.88675 64.29375) (width 0.2) (layer "F.Cu") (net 10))
 (segment (start 114.88675 64.29375) (end 128.905 64.29375) (width 0.2) (layer "F.Cu") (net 10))
 (segment (start 128.905 64.29375) (end 129.06375 64.4525) (width 0.2) (layer "F.Cu") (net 10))
 (segment (start 111.47175 64.29375) (end 111.47175 63.650874) (width 0.2) (layer "F.Cu") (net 10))
 (segment (start 139.02125 89.65) (end 139.05875 89.65) (width 0.2) (layer "F.Cu") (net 8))
 (segment (start 113.82375 64.4525) (end 139.02125 89.65) (width 0.2) (layer "F.Cu") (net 8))
 (segment (start 139.53551 90.801) (end 140.20975 90.12676) (width 0.2) (layer "F.Cu") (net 7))
 (segment (start 140.20975 90.12676) (end 140.20975 88.261) (width 0.2) (layer "F.Cu") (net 7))
 (segment (start 140.20975 88.261) (end 139.05875 87.11) (width 0.2) (layer "F.Cu") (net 7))
 (segment (start 137.63225 90.801) (end 139.53551 90.801) (width 0.2) (layer "F.Cu") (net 7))
 (segment (start 113.82375 66.9925) (end 137.63225 90.801) (width 0.2) (layer "F.Cu") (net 7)))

